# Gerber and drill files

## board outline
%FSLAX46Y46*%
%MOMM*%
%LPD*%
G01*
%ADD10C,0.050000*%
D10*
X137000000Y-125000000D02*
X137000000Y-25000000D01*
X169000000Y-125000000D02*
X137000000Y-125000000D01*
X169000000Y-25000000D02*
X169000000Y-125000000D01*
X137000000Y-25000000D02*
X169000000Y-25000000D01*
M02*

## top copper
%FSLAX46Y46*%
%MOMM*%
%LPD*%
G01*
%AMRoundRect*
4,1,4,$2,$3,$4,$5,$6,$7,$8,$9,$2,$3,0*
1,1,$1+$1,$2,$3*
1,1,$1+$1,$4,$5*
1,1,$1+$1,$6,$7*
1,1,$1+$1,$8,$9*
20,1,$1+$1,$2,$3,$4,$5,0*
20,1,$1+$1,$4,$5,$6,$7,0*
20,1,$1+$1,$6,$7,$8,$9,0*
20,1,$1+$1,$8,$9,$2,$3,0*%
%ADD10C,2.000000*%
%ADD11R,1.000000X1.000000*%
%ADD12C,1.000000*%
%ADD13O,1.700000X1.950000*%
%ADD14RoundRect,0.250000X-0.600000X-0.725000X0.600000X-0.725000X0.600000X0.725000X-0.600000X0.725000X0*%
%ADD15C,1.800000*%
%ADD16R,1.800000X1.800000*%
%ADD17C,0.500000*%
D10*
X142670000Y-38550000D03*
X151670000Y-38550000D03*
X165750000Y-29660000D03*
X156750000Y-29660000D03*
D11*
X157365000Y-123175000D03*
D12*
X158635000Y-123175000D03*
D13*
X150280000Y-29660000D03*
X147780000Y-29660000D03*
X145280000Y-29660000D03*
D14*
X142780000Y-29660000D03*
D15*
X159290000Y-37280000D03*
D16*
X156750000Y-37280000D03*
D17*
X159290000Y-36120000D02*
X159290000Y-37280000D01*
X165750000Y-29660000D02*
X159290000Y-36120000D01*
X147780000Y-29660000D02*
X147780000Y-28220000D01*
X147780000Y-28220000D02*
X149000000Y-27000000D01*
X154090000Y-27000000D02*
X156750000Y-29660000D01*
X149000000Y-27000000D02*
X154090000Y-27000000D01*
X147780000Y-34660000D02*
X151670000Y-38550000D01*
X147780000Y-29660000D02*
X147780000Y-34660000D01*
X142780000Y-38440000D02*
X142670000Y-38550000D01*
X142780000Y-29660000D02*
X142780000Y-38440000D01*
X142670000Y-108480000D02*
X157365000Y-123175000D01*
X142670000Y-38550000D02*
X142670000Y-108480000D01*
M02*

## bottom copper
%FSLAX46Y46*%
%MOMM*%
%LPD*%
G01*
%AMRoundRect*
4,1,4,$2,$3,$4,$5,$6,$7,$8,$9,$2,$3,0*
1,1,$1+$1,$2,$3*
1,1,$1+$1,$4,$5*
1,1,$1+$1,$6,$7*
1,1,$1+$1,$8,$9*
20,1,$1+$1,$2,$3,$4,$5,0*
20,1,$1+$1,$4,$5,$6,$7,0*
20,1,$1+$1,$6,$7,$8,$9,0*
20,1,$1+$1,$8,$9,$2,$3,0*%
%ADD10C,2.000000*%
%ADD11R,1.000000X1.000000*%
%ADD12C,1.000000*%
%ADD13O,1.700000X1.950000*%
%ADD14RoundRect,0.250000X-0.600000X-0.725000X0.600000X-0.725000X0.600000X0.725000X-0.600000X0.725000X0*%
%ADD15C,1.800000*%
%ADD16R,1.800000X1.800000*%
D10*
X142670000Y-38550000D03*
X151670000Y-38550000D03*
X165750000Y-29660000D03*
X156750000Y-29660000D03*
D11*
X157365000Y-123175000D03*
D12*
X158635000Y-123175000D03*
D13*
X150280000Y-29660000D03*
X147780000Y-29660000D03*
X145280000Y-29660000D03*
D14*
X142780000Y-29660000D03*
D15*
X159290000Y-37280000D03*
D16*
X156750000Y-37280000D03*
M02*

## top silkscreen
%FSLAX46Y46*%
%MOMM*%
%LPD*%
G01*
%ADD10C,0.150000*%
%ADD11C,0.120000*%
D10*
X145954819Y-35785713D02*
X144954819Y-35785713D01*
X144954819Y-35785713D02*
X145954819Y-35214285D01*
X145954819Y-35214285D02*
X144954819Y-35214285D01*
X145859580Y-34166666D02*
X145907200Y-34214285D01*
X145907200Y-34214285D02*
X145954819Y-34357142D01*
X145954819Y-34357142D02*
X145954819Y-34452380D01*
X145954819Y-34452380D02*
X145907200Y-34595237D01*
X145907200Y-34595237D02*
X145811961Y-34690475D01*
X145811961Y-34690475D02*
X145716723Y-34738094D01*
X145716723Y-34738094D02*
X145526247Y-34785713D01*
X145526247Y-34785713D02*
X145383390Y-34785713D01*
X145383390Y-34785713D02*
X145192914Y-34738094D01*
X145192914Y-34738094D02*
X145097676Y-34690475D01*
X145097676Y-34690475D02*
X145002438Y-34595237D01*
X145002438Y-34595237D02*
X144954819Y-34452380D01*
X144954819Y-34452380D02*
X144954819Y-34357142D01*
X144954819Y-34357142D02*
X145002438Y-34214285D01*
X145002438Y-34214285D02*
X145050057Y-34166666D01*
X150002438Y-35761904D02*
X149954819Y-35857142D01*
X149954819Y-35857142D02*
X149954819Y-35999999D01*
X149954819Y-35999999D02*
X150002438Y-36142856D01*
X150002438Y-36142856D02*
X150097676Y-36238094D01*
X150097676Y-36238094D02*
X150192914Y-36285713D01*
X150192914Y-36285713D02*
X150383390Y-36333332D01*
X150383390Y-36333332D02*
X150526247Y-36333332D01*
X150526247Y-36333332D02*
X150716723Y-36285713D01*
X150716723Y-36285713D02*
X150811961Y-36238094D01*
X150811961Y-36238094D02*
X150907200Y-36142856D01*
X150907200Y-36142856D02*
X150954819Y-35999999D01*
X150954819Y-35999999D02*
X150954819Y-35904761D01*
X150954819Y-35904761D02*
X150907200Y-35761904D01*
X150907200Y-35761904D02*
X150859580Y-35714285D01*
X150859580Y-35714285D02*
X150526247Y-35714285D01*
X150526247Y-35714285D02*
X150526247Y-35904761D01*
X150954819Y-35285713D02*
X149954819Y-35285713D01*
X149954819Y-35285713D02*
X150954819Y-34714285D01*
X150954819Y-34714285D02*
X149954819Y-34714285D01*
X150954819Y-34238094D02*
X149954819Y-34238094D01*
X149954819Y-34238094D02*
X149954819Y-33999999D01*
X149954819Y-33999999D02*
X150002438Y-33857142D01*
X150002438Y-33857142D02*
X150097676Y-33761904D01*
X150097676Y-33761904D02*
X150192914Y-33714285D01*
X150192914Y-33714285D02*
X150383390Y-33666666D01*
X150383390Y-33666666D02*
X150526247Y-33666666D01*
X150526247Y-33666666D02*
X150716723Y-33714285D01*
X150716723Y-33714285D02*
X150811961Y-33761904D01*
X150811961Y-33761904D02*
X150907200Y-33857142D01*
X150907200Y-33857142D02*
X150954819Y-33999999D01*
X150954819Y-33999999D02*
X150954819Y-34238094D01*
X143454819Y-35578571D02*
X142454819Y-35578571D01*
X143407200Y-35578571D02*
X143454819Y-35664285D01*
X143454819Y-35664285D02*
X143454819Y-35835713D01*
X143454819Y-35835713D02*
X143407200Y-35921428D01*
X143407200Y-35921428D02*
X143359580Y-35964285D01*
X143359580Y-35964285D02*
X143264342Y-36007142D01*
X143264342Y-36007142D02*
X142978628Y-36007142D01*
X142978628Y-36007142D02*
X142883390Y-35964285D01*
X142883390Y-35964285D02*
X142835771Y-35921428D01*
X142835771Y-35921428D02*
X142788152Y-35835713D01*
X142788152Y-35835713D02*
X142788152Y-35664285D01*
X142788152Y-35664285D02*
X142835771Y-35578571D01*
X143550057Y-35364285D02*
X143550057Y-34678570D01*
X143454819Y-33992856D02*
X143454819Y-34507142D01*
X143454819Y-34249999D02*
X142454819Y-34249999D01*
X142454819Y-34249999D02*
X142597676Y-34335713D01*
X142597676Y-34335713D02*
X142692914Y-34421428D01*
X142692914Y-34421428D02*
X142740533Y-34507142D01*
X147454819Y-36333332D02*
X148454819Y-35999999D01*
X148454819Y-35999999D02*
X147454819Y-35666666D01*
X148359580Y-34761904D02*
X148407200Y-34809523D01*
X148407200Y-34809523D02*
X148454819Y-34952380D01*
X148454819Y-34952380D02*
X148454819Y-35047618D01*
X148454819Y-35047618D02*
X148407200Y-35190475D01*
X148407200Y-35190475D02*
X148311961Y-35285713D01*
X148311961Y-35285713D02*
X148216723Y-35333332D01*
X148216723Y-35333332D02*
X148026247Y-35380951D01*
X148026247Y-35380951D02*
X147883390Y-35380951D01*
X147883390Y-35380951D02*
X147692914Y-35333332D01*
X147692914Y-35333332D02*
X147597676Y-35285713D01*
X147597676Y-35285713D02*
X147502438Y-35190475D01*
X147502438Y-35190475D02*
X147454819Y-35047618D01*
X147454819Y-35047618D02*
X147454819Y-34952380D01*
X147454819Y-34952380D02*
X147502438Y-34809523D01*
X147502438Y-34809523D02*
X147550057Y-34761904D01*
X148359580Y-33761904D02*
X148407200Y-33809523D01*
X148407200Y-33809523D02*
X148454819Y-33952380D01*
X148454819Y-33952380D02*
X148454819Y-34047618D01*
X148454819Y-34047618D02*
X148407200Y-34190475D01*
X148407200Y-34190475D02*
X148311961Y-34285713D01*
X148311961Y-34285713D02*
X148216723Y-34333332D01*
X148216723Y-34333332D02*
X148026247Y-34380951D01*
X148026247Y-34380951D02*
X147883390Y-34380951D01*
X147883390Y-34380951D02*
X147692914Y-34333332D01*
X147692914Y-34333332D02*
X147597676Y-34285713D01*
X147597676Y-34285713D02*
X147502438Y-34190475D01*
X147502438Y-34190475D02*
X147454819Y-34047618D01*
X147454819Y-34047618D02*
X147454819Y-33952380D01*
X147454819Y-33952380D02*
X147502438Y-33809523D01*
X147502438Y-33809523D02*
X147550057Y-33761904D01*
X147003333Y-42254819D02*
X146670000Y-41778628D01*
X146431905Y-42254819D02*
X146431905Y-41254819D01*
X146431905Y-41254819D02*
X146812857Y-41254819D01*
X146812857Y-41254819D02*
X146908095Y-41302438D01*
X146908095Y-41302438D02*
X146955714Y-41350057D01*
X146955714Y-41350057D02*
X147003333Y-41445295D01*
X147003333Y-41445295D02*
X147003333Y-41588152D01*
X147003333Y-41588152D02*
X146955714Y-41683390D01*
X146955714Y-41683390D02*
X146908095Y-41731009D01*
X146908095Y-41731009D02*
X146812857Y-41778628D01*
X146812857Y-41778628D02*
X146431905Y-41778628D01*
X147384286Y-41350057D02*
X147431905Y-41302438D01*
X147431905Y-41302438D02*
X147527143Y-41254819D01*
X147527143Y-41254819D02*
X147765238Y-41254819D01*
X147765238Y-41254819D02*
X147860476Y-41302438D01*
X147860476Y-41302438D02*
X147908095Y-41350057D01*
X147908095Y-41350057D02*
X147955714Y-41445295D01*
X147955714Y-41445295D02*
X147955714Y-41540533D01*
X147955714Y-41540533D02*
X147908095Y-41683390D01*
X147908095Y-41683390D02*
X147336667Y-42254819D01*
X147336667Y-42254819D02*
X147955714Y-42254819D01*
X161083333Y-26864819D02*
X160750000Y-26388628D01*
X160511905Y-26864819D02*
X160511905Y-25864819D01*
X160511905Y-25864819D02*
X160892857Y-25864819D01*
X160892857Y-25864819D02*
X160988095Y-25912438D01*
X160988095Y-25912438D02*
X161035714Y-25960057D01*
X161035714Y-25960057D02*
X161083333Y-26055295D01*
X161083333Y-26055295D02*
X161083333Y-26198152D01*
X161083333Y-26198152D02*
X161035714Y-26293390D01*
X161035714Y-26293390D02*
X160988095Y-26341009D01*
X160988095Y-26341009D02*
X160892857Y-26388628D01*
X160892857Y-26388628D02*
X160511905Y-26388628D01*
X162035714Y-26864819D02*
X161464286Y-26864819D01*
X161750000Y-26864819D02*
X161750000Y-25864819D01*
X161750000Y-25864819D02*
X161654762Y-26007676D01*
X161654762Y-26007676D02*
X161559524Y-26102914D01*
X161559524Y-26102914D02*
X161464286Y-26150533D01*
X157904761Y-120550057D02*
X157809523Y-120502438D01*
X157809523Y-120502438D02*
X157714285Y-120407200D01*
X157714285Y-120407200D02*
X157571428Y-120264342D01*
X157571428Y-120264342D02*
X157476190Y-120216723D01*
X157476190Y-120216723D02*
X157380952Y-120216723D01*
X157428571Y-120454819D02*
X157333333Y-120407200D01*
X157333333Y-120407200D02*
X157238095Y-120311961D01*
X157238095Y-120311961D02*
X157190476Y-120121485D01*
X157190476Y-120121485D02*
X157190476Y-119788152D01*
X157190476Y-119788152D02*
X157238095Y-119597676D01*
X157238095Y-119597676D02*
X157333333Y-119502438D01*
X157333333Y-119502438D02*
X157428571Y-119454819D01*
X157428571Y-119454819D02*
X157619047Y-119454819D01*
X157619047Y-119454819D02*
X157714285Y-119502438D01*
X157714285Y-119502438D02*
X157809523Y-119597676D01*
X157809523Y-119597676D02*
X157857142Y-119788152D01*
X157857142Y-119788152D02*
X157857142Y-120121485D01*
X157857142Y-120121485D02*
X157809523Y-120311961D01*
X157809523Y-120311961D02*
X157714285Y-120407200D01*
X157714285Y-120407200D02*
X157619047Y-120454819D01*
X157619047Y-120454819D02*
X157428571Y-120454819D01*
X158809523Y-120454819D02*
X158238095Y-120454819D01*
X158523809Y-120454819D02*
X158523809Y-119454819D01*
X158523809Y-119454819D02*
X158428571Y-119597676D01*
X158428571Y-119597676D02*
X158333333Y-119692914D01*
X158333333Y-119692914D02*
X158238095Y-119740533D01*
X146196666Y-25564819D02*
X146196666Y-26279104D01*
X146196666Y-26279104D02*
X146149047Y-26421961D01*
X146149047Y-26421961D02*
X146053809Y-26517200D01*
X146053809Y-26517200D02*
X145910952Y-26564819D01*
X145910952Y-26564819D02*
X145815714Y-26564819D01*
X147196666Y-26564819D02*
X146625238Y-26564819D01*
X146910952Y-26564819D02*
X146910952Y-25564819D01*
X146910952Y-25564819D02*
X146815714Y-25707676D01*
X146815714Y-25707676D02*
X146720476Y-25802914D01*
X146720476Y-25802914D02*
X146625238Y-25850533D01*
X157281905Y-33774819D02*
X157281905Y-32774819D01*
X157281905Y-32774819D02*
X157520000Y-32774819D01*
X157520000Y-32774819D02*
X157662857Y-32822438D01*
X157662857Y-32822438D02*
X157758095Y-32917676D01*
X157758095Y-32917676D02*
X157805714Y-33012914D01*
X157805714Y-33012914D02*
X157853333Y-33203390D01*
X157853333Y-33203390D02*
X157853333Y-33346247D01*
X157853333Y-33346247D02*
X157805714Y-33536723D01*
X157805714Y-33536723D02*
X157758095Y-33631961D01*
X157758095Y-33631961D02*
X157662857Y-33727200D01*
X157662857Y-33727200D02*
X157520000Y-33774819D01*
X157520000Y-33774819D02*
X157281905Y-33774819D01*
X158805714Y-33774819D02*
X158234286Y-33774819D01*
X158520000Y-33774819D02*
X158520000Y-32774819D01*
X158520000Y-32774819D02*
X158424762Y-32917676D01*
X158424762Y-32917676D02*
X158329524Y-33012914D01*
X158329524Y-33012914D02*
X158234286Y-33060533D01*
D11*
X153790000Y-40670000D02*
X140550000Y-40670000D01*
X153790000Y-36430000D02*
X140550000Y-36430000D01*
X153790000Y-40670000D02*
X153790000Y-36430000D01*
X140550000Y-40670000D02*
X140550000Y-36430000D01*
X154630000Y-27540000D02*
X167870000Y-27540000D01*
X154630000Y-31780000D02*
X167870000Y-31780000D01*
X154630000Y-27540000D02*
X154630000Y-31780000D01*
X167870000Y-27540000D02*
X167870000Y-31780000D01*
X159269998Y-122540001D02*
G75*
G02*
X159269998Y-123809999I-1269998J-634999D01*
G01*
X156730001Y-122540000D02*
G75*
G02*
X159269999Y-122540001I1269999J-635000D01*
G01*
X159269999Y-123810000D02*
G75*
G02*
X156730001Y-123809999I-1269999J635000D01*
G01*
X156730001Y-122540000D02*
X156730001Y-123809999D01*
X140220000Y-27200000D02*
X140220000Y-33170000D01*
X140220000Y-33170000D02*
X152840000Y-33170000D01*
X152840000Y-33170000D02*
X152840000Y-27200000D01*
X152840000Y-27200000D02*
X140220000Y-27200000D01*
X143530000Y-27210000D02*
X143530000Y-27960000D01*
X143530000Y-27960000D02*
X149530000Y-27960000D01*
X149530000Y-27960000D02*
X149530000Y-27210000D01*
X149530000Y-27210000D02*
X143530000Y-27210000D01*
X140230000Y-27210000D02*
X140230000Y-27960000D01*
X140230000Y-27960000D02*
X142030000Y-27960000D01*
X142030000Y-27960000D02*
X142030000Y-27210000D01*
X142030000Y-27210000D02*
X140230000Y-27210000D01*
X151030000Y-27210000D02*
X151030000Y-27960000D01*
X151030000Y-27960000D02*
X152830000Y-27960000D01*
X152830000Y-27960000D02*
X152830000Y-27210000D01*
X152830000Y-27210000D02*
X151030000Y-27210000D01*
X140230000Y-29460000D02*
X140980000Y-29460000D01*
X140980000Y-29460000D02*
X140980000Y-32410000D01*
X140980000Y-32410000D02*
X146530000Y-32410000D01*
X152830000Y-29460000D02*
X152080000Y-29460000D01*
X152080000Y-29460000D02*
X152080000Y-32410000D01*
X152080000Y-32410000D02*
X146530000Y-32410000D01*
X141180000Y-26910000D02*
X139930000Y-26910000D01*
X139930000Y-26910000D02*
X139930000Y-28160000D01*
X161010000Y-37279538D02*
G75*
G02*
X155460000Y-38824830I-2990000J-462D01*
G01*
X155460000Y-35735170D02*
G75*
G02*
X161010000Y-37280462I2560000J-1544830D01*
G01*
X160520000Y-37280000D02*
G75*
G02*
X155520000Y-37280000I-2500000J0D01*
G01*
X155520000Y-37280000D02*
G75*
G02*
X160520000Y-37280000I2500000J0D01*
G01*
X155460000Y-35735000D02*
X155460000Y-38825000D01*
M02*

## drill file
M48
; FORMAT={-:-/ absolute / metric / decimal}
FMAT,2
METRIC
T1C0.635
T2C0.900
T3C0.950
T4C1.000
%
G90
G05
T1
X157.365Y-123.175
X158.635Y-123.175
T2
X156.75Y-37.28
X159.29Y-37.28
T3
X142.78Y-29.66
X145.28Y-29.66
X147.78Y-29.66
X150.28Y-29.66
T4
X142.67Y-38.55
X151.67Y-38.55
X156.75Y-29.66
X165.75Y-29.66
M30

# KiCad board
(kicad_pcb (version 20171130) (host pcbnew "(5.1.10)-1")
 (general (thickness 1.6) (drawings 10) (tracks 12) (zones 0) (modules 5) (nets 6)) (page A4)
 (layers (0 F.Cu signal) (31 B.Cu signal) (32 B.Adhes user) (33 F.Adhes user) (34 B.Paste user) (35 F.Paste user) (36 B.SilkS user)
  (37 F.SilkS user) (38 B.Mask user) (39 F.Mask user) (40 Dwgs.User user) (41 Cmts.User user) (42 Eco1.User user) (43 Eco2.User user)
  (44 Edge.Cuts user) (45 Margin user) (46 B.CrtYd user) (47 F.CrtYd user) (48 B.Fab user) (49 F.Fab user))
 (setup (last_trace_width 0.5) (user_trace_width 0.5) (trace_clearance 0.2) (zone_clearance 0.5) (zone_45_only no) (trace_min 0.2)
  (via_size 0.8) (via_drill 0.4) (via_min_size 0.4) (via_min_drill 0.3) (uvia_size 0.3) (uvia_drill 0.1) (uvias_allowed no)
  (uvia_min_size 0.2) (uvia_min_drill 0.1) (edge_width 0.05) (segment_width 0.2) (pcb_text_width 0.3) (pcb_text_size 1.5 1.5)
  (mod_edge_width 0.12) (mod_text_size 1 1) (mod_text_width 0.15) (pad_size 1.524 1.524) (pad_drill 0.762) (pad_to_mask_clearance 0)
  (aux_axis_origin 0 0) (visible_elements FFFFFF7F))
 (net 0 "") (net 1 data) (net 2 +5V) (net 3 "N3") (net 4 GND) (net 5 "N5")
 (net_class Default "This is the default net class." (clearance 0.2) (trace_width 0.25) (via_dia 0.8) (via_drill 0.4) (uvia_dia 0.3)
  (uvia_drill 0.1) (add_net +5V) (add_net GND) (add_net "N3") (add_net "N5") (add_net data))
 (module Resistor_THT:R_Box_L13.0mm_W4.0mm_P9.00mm (layer F.Cu) (at 151.67 38.55 180)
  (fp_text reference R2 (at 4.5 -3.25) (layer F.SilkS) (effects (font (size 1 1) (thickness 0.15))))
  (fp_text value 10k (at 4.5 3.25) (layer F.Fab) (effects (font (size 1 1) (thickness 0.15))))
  (fp_line (start -2.12 -2.12) (end 11.12 -2.12) (layer F.SilkS) (width 0.12))
  (fp_line (start -2.12 2.12) (end 11.12 2.12) (layer F.SilkS) (width 0.12))
  (fp_line (start -2.12 -2.12) (end -2.12 2.12) (layer F.SilkS) (width 0.12))
  (fp_line (start 11.12 -2.12) (end 11.12 2.12) (layer F.SilkS) (width 0.12))
  (pad 2 thru_hole circle (at 9 0 180) (size 2 2) (drill 1) (layers *.Cu *.Mask) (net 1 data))
  (pad 1 thru_hole circle (at 0 0 180) (size 2 2) (drill 1) (layers *.Cu *.Mask) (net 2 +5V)))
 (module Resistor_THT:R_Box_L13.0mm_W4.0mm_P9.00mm (layer F.Cu) (at 156.75 29.66)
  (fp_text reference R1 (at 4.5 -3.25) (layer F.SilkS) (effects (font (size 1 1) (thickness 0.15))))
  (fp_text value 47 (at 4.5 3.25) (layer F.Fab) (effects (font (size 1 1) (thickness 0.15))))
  (fp_line (start -2.12 -2.12) (end 11.12 -2.12) (layer F.SilkS) (width 0.12))
  (fp_line (start -2.12 2.12) (end 11.12 2.12) (layer F.SilkS) (width 0.12))
  (fp_line (start -2.12 -2.12) (end -2.12 2.12) (layer F.SilkS) (width 0.12))
  (fp_line (start 11.12 -2.12) (end 11.12 2.12) (layer F.SilkS) (width 0.12))
  (pad 2 thru_hole circle (at 9 0) (size 2 2) (drill 1) (layers *.Cu *.Mask) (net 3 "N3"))
  (pad 1 thru_hole circle (at 0 0) (size 2 2) (drill 1) (layers *.Cu *.Mask) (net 2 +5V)))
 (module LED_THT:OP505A (layer F.Cu) (at 158 120)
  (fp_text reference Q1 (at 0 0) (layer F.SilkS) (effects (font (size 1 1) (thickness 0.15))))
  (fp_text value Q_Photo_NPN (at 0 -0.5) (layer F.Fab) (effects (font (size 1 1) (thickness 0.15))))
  (fp_arc (start 0 3.175) (end 1.269998 3.809999) (angle -53.13010235) (layer F.SilkS) (width 0.12))
  (fp_arc (start 0 3.175) (end 1.269999 2.540001) (angle -126.8698976) (layer F.SilkS) (width 0.12))
  (fp_arc (start 0 3.175) (end -1.269999 3.809999) (angle -126.8698976) (layer F.SilkS) (width 0.12))
  (fp_line (start -1.269999 2.54) (end -1.269999 3.809999) (layer F.SilkS) (width 0.12))
  (pad 1 thru_hole rect (at -0.635 3.175) (size 1 1) (drill 0.635) (layers *.Cu *.Mask) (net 1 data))
  (pad 2 thru_hole circle (at 0.635 3.175) (size 1 1) (drill 0.635) (layers *.Cu *.Mask)))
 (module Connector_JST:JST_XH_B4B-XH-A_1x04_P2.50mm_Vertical (layer F.Cu) (at 142.78 29.66)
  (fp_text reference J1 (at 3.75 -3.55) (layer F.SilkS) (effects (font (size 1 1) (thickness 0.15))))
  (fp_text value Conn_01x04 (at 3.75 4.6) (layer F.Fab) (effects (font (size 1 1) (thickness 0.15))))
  (fp_line (start -2.56 -2.46) (end -2.56 3.51) (layer F.SilkS) (width 0.12))
  (fp_line (start -2.56 3.51) (end 10.06 3.51) (layer F.SilkS) (width 0.12))
  (fp_line (start 10.06 3.51) (end 10.06 -2.46) (layer F.SilkS) (width 0.12))
  (fp_line (start 10.06 -2.46) (end -2.56 -2.46) (layer F.SilkS) (width 0.12))
  (fp_line (start 0.75 -2.45) (end 0.75 -1.7) (layer F.SilkS) (width 0.12))
  (fp_line (start 0.75 -1.7) (end 6.75 -1.7) (layer F.SilkS) (width 0.12))
  (fp_line (start 6.75 -1.7) (end 6.75 -2.45) (layer F.SilkS) (width 0.12))
  (fp_line (start 6.75 -2.45) (end 0.75 -2.45) (layer F.SilkS) (width 0.12))
  (fp_line (start -2.55 -2.45) (end -2.55 -1.7) (layer F.SilkS) (width 0.12))
  (fp_line (start -2.55 -1.7) (end -0.75 -1.7) (layer F.SilkS) (width 0.12))
  (fp_line (start -0.75 -1.7) (end -0.75 -2.45) (layer F.SilkS) (width 0.12))
  (fp_line (start -0.75 -2.45) (end -2.55 -2.45) (layer F.SilkS) (width 0.12))
  (fp_line (start 8.25 -2.45) (end 8.25 -1.7) (layer F.SilkS) (width 0.12))
  (fp_line (start 8.25 -1.7) (end 10.05 -1.7) (layer F.SilkS) (width 0.12))
  (fp_line (start 10.05 -1.7) (end 10.05 -2.45) (layer F.SilkS) (width 0.12))
  (fp_line (start 10.05 -2.45) (end 8.25 -2.45) (layer F.SilkS) (width 0.12))
  (fp_line (start -2.55 -0.2) (end -1.8 -0.2) (layer F.SilkS) (width 0.12))
  (fp_line (start -1.8 -0.2) (end -1.8 2.75) (layer F.SilkS) (width 0.12))
  (fp_line (start -1.8 2.75) (end 3.75 2.75) (layer F.SilkS) (width 0.12))
  (fp_line (start 10.05 -0.2) (end 9.3 -0.2) (layer F.SilkS) (width 0.12))
  (fp_line (start 9.3 -0.2) (end 9.3 2.75) (layer F.SilkS) (width 0.12))
  (fp_line (start 9.3 2.75) (end 3.75 2.75) (layer F.SilkS) (width 0.12))
  (fp_line (start -1.6 -2.75) (end -2.85 -2.75) (layer F.SilkS) (width 0.12))
  (fp_line (start -2.85 -2.75) (end -2.85 -1.5) (layer F.SilkS) (width 0.12))
  (pad 4 thru_hole oval (at 7.5 0) (size 1.7 1.95) (drill 0.95) (layers *.Cu *.Mask))
  (pad 3 thru_hole oval (at 5 0) (size 1.7 1.95) (drill 0.95) (layers *.Cu *.Mask) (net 2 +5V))
  (pad 2 thru_hole oval (at 2.5 0) (size 1.7 1.95) (drill 0.95) (layers *.Cu *.Mask))
  (pad 1 thru_hole roundrect (at 0 0) (size 1.7 1.95) (drill 0.95) (layers *.Cu *.Mask) (roundrect_rratio 0.1470588235294118) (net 1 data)))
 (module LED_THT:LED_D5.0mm (layer F.Cu) (at 156.75 37.28)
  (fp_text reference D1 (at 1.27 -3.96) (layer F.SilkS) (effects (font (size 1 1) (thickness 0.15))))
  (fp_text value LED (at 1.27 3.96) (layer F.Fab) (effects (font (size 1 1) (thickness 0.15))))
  (fp_arc (start 1.27 0) (end -1.29 1.54483) (angle -148.9) (layer F.SilkS) (width 0.12))
  (fp_arc (start 1.27 0) (end -1.29 -1.54483) (angle 148.9) (layer F.SilkS) (width 0.12))
  (fp_circle (center 1.27 0) (end 3.77 0) (layer F.SilkS) (width 0.12))
  (fp_line (start -1.29 -1.545) (end -1.29 1.545) (layer F.SilkS) (width 0.12))
  (pad 2 thru_hole circle (at 2.54 0) (size 1.8 1.8) (drill 0.9) (layers *.Cu *.Mask) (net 3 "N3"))
  (pad 1 thru_hole rect (at 0 0) (size 1.8 1.8) (drill 0.9) (layers *.Cu *.Mask)))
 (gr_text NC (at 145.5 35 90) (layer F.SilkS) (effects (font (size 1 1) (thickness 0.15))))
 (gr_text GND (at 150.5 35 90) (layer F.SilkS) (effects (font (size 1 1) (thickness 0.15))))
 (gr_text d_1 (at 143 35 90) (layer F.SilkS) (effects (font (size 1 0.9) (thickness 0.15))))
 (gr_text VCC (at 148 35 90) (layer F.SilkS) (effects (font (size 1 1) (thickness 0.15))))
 (gr_line (start 137 125) (end 137 25) (layer Edge.Cuts) (width 0.05))
 (gr_line (start 169 125) (end 137 125) (layer Edge.Cuts) (width 0.05))
 (gr_line (start 169 25) (end 169 125) (layer Edge.Cuts) (width 0.05))
 (gr_line (start 137 25) (end 169 25) (layer Edge.Cuts) (width 0.05))
 (segment (start 159.29 36.12) (end 159.29 37.28) (width 0.5) (layer F.Cu) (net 3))
 (segment (start 165.75 29.66) (end 159.29 36.12) (width 0.5) (layer F.Cu) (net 3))
 (segment (start 147.78 29.66) (end 147.78 28.22) (width 0.5) (layer F.Cu) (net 2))
 (segment (start 147.78 28.22) (end 149 27) (width 0.5) (layer F.Cu) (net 2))
 (segment (start 154.09 27) (end 156.75 29.66) (width 0.5) (layer F.Cu) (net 2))
 (segment (start 149 27) (end 154.09 27) (width 0.5) (layer F.Cu) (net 2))
 (segment (start 147.78 34.66) (end 151.67 38.55) (width 0.5) (layer F.Cu) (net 2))
 (segment (start 147.78 29.66) (end 147.78 34.66) (width 0.5) (layer F.Cu) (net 2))
 (segment (start 142.78 38.44) (end 142.67 38.55) (width 0.5) (layer F.Cu) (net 1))
 (segment (start 142.78 29.66) (end 142.78 38.44) (width 0.5) (layer F.Cu) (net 1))
 (segment (start 142.67 108.48) (end 157.365 123.175) (width 0.5) (layer F.Cu) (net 1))
 (segment (start 142.67 38.55) (end 142.67 108.48) (width 0.5) (layer F.Cu) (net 1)))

